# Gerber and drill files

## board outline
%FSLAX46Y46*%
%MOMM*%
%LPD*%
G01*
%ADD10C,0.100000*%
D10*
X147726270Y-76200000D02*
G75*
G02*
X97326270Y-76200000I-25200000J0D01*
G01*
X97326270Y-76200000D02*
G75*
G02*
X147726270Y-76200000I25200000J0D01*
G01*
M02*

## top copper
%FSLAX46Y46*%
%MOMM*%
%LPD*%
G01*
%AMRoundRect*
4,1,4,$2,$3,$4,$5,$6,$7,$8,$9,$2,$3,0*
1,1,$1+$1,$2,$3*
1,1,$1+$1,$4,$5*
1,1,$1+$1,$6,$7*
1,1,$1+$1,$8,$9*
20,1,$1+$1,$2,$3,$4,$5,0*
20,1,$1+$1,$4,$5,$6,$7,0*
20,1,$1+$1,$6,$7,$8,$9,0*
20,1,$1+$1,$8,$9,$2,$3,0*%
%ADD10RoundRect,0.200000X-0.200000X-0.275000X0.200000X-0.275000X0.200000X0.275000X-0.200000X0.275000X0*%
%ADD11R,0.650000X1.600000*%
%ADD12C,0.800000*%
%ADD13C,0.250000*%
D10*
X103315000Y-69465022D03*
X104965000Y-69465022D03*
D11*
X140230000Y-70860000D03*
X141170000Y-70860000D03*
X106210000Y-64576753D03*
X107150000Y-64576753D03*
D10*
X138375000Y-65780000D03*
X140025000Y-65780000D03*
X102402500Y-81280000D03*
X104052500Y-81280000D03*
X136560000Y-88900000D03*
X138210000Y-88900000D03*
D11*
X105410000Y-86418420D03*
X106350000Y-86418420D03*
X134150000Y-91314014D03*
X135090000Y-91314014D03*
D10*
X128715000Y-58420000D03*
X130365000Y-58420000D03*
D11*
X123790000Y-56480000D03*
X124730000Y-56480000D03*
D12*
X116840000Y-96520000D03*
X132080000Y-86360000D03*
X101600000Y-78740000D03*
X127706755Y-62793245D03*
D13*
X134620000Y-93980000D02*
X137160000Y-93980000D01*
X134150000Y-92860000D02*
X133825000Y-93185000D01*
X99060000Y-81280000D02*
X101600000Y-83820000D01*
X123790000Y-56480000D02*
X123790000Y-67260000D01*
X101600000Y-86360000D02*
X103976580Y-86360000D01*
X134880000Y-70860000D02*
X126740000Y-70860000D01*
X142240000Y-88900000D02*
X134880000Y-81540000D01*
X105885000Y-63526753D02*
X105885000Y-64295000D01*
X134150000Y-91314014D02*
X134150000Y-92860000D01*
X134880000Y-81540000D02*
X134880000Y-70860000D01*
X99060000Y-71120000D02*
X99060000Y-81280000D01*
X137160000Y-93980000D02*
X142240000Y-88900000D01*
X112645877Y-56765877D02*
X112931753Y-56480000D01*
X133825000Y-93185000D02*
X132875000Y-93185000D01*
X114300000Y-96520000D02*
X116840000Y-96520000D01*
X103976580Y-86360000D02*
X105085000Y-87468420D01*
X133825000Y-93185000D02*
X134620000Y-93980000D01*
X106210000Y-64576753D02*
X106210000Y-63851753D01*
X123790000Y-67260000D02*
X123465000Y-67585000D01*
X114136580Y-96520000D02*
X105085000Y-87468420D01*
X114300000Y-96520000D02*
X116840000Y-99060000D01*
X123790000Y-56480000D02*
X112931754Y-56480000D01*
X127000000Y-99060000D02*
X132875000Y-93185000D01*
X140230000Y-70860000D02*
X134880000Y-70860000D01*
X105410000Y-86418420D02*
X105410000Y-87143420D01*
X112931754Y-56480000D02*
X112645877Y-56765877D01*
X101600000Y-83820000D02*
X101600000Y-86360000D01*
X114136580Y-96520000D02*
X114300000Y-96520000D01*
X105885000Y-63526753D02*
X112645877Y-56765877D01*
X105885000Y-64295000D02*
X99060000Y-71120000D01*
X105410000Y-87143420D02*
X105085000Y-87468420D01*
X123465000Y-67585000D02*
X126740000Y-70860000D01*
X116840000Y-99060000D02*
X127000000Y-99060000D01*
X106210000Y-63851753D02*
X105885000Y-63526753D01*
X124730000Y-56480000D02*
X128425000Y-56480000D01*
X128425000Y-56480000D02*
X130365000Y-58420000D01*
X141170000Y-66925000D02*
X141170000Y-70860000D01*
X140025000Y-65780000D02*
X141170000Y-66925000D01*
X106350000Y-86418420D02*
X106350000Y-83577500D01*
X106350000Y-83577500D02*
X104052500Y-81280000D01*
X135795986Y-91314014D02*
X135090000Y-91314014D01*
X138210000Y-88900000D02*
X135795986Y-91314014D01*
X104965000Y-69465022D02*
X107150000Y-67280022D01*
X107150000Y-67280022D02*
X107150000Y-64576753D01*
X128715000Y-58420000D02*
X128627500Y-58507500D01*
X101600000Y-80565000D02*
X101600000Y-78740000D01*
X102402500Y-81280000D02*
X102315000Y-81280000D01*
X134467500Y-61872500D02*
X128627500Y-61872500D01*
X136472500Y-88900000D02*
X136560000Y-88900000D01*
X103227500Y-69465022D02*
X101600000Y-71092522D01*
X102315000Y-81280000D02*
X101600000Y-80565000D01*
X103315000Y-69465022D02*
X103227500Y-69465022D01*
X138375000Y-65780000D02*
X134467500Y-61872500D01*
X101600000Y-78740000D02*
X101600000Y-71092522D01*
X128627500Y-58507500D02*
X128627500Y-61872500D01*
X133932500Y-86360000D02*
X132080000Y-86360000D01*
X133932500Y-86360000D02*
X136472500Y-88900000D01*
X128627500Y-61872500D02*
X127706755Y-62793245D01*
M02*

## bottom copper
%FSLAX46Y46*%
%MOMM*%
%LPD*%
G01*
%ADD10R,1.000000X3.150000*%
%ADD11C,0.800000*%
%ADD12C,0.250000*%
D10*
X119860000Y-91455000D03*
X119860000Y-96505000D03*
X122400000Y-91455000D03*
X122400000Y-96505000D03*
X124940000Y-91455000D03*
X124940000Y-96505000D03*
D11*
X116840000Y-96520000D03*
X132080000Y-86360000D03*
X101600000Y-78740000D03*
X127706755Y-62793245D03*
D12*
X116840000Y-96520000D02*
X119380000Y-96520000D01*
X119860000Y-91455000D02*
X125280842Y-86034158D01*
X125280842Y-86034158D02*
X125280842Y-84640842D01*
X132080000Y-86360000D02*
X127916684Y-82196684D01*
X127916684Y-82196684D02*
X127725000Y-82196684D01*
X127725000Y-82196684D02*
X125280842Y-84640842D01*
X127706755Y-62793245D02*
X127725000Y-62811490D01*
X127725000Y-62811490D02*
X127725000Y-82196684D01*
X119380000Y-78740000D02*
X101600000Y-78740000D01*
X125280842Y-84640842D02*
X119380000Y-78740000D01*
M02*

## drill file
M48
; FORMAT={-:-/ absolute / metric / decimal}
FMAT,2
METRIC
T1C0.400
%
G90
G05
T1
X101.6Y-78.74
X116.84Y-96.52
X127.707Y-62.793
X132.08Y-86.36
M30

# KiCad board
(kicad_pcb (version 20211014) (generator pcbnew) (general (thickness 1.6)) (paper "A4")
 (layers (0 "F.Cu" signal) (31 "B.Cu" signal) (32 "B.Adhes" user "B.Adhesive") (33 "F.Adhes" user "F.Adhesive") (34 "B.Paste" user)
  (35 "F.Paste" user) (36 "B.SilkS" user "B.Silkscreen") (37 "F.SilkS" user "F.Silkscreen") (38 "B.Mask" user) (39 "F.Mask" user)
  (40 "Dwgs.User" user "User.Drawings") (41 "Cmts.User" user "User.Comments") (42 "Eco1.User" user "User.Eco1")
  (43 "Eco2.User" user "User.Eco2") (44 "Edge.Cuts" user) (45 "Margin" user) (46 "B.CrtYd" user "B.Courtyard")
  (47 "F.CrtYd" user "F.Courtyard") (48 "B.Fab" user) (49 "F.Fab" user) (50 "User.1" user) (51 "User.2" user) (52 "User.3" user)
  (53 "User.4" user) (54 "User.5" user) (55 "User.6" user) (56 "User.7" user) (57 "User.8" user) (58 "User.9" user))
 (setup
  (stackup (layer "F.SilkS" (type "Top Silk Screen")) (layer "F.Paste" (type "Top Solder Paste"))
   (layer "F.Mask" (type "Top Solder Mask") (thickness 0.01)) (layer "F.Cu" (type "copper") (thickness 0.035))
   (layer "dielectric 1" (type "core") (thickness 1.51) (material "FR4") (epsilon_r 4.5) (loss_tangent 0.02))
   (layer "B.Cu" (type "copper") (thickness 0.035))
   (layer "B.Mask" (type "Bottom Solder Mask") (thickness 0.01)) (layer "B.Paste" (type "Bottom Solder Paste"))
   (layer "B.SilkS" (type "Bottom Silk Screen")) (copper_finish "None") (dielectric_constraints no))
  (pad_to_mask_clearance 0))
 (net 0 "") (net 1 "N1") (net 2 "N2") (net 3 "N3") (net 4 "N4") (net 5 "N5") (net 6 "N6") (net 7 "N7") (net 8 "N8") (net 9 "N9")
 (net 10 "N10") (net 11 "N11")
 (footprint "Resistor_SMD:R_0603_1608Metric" (layer "F.Cu") (at 104.14 69.465022)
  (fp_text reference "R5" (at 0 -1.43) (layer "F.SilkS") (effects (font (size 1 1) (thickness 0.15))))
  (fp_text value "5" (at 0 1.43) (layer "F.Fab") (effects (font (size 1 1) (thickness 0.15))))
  (pad "1" smd roundrect (at -0.825 0) (size 0.8 0.95) (layers "F.Cu" "F.Paste" "F.Mask") (roundrect_rratio 0.25) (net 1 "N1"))
  (pad "2" smd roundrect (at 0.825 0) (size 0.8 0.95) (layers "F.Cu" "F.Paste" "F.Mask") (roundrect_rratio 0.25) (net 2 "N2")))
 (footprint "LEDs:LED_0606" (layer "F.Cu") (at 140.7 70.86)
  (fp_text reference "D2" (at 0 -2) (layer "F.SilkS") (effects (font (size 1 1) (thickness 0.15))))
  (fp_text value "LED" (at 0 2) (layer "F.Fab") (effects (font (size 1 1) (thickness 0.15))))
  (pad "1" smd rect locked (at -0.47 0 180) (size 0.65 1.6) (layers "F.Cu" "F.Paste" "F.Mask") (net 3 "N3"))
  (pad "2" smd rect locked (at 0.47 0 180) (size 0.65 1.6) (layers "F.Cu" "F.Paste" "F.Mask") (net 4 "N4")))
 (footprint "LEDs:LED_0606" (layer "F.Cu") (at 106.68 64.576753)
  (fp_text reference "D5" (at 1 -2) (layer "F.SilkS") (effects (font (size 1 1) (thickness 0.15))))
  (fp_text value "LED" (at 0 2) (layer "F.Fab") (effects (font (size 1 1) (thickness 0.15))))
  (pad "1" smd rect locked (at -0.47 0 180) (size 0.65 1.6) (layers "F.Cu" "F.Paste" "F.Mask") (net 3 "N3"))
  (pad "2" smd rect locked (at 0.47 0 180) (size 0.65 1.6) (layers "F.Cu" "F.Paste" "F.Mask") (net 2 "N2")))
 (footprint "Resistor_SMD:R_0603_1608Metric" (layer "F.Cu") (at 139.2 65.78)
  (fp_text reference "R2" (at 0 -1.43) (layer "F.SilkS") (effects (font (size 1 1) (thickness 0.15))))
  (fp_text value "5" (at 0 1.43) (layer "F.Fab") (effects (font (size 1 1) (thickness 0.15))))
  (pad "1" smd roundrect (at -0.825 0) (size 0.8 0.95) (layers "F.Cu" "F.Paste" "F.Mask") (roundrect_rratio 0.25) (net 1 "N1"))
  (pad "2" smd roundrect (at 0.825 0) (size 0.8 0.95) (layers "F.Cu" "F.Paste" "F.Mask") (roundrect_rratio 0.25) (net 4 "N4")))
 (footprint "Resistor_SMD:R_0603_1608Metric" (layer "F.Cu") (at 103.2275 81.28)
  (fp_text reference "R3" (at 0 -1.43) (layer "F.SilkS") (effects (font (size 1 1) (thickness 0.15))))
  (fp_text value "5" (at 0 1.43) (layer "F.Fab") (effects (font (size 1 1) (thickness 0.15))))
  (pad "1" smd roundrect (at -0.825 0) (size 0.8 0.95) (layers "F.Cu" "F.Paste" "F.Mask") (roundrect_rratio 0.25) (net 1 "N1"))
  (pad "2" smd roundrect (at 0.825 0) (size 0.8 0.95) (layers "F.Cu" "F.Paste" "F.Mask") (roundrect_rratio 0.25) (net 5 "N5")))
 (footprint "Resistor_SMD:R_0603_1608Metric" (layer "F.Cu") (at 137.385 88.9)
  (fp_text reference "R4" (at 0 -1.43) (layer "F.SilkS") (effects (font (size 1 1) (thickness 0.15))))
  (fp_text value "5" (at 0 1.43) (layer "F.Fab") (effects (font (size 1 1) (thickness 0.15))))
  (pad "1" smd roundrect (at -0.825 0) (size 0.8 0.95) (layers "F.Cu" "F.Paste" "F.Mask") (roundrect_rratio 0.25) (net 1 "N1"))
  (pad "2" smd roundrect (at 0.825 0) (size 0.8 0.95) (layers "F.Cu" "F.Paste" "F.Mask") (roundrect_rratio 0.25) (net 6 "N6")))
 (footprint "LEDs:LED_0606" (layer "F.Cu") (at 105.88 86.41842)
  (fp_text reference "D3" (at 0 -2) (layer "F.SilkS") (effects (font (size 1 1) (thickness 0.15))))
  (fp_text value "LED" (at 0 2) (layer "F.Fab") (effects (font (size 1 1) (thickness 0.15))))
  (pad "1" smd rect locked (at -0.47 0 180) (size 0.65 1.6) (layers "F.Cu" "F.Paste" "F.Mask") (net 3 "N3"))
  (pad "2" smd rect locked (at 0.47 0 180) (size 0.65 1.6) (layers "F.Cu" "F.Paste" "F.Mask") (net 5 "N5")))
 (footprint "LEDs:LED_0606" (layer "F.Cu") (at 134.62 91.314014)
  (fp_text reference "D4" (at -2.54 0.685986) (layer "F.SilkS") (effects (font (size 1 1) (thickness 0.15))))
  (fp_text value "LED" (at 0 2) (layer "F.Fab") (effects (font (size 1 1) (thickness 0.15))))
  (pad "1" smd rect locked (at -0.47 0 180) (size 0.65 1.6) (layers "F.Cu" "F.Paste" "F.Mask") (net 3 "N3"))
  (pad "2" smd rect locked (at 0.47 0 180) (size 0.65 1.6) (layers "F.Cu" "F.Paste" "F.Mask") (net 6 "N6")))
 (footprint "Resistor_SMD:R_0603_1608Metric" (layer "F.Cu") (at 129.54 58.42)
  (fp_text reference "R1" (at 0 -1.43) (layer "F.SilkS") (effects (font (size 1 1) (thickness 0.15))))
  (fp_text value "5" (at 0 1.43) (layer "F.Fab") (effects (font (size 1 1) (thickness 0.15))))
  (pad "1" smd roundrect (at -0.825 0) (size 0.8 0.95) (layers "F.Cu" "F.Paste" "F.Mask") (roundrect_rratio 0.25) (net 1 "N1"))
  (pad "2" smd roundrect (at 0.825 0) (size 0.8 0.95) (layers "F.Cu" "F.Paste" "F.Mask") (roundrect_rratio 0.25) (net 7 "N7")))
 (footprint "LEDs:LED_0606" (layer "F.Cu") (at 124.26 56.48)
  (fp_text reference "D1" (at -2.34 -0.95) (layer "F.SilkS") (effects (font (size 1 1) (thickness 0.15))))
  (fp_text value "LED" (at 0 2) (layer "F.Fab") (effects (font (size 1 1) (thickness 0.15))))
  (pad "1" smd rect locked (at -0.47 0 180) (size 0.65 1.6) (layers "F.Cu" "F.Paste" "F.Mask") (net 3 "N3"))
  (pad "2" smd rect locked (at 0.47 0 180) (size 0.65 1.6) (layers "F.Cu" "F.Paste" "F.Mask") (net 7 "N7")))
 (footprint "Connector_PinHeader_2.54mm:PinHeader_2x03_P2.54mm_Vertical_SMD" (layer "B.Cu") (at 122.4 93.98 -90)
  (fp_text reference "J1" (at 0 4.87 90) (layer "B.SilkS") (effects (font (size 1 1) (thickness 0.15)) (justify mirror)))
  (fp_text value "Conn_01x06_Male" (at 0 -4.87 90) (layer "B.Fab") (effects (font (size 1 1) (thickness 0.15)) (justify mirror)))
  (pad "1" smd rect (at -2.525 2.54 270) (size 3.15 1) (layers "B.Cu" "B.Paste" "B.Mask") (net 1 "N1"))
  (pad "2" smd rect (at 2.525 2.54 270) (size 3.15 1) (layers "B.Cu" "B.Paste" "B.Mask") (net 3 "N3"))
  (pad "3" smd rect (at -2.525 0 270) (size 3.15 1) (layers "B.Cu" "B.Paste" "B.Mask") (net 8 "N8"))
  (pad "4" smd rect (at 2.525 0 270) (size 3.15 1) (layers "B.Cu" "B.Paste" "B.Mask") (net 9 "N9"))
  (pad "5" smd rect (at -2.525 -2.54 270) (size 3.15 1) (layers "B.Cu" "B.Paste" "B.Mask") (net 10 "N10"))
  (pad "6" smd rect (at 2.525 -2.54 270) (size 3.15 1) (layers "B.Cu" "B.Paste" "B.Mask") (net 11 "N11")))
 (gr_circle (center 122.52627 76.2) (end 147.72627 76.2) (layer "Edge.Cuts") (width 0.1) (fill none))
 (segment (start 134.62 93.98) (end 137.16 93.98) (width 0.25) (layer "F.Cu") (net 3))
 (segment (start 134.15 92.86) (end 133.825 93.185) (width 0.25) (layer "F.Cu") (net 3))
 (segment (start 99.06 81.28) (end 101.6 83.82) (width 0.25) (layer "F.Cu") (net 3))
 (segment (start 123.79 56.48) (end 123.79 67.26) (width 0.25) (layer "F.Cu") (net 3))
 (segment (start 101.6 86.36) (end 103.97658 86.36) (width 0.25) (layer "F.Cu") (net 3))
 (segment (start 134.88 70.86) (end 126.74 70.86) (width 0.25) (layer "F.Cu") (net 3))
 (segment (start 142.24 88.9) (end 134.88 81.54) (width 0.25) (layer "F.Cu") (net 3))
 (segment (start 105.885 63.526753) (end 105.885 64.295) (width 0.25) (layer "F.Cu") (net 3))
 (segment (start 134.15 91.314014) (end 134.15 92.86) (width 0.25) (layer "F.Cu") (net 3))
 (segment (start 134.88 81.54) (end 134.88 70.86) (width 0.25) (layer "F.Cu") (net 3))
 (segment (start 99.06 71.12) (end 99.06 81.28) (width 0.25) (layer "F.Cu") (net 3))
 (segment (start 137.16 93.98) (end 142.24 88.9) (width 0.25) (layer "F.Cu") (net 3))
 (segment (start 112.645877 56.765877) (end 112.931753 56.48) (width 0.25) (layer "F.Cu") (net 3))
 (segment (start 133.825 93.185) (end 132.875 93.185) (width 0.25) (layer "F.Cu") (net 3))
 (segment (start 114.3 96.52) (end 116.84 96.52) (width 0.25) (layer "F.Cu") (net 3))
 (segment (start 103.97658 86.36) (end 105.085 87.46842) (width 0.25) (layer "F.Cu") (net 3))
 (segment (start 133.825 93.185) (end 134.62 93.98) (width 0.25) (layer "F.Cu") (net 3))
 (segment (start 106.21 64.576753) (end 106.21 63.851753) (width 0.25) (layer "F.Cu") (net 3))
 (segment (start 123.79 67.26) (end 123.465 67.585) (width 0.25) (layer "F.Cu") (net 3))
 (segment (start 114.13658 96.52) (end 105.085 87.46842) (width 0.25) (layer "F.Cu") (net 3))
 (segment (start 114.3 96.52) (end 116.84 99.06) (width 0.25) (layer "F.Cu") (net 3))
 (segment (start 123.79 56.48) (end 112.931754 56.48) (width 0.25) (layer "F.Cu") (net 3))
 (segment (start 127 99.06) (end 132.875 93.185) (width 0.25) (layer "F.Cu") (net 3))
 (segment (start 140.23 70.86) (end 134.88 70.86) (width 0.25) (layer "F.Cu") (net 3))
 (segment (start 105.41 86.41842) (end 105.41 87.14342) (width 0.25) (layer "F.Cu") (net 3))
 (segment (start 112.931754 56.48) (end 112.645877 56.765877) (width 0.25) (layer "F.Cu") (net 3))
 (segment (start 101.6 83.82) (end 101.6 86.36) (width 0.25) (layer "F.Cu") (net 3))
 (segment (start 114.13658 96.52) (end 114.3 96.52) (width 0.25) (layer "F.Cu") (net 3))
 (segment (start 105.885 63.526753) (end 112.645877 56.765877) (width 0.25) (layer "F.Cu") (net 3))
 (segment (start 105.885 64.295) (end 99.06 71.12) (width 0.25) (layer "F.Cu") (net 3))
 (segment (start 105.41 87.14342) (end 105.085 87.46842) (width 0.25) (layer "F.Cu") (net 3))
 (segment (start 123.465 67.585) (end 126.74 70.86) (width 0.25) (layer "F.Cu") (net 3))
 (segment (start 116.84 99.06) (end 127 99.06) (width 0.25) (layer "F.Cu") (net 3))
 (segment (start 106.21 63.851753) (end 105.885 63.526753) (width 0.25) (layer "F.Cu") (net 3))
 (via (at 116.84 96.52) (size 0.8) (drill 0.4) (layers "F.Cu" "B.Cu") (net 3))
 (segment (start 116.84 96.52) (end 119.38 96.52) (width 0.25) (layer "B.Cu") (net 3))
 (segment (start 124.73 56.48) (end 128.425 56.48) (width 0.25) (layer "F.Cu") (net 7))
 (segment (start 128.425 56.48) (end 130.365 58.42) (width 0.25) (layer "F.Cu") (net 7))
 (segment (start 141.17 66.925) (end 141.17 70.86) (width 0.25) (layer "F.Cu") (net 4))
 (segment (start 140.025 65.78) (end 141.17 66.925) (width 0.25) (layer "F.Cu") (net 4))
 (segment (start 106.35 86.41842) (end 106.35 83.5775) (width 0.25) (layer "F.Cu") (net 5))
 (segment (start 106.35 83.5775) (end 104.0525 81.28) (width 0.25) (layer "F.Cu") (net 5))
 (segment (start 135.795986 91.314014) (end 135.09 91.314014) (width 0.25) (layer "F.Cu") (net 6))
 (segment (start 138.21 88.9) (end 135.795986 91.314014) (width 0.25) (layer "F.Cu") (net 6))
 (segment (start 104.965 69.465022) (end 107.15 67.280022) (width 0.25) (layer "F.Cu") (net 2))
 (segment (start 107.15 67.280022) (end 107.15 64.576753) (width 0.25) (layer "F.Cu") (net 2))
 (segment (start 128.715 58.42) (end 128.6275 58.5075) (width 0.25) (layer "F.Cu") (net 1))
 (segment (start 101.6 80.565) (end 101.6 78.74) (width 0.25) (layer "F.Cu") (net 1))
 (segment (start 102.4025 81.28) (end 102.315 81.28) (width 0.25) (layer "F.Cu") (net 1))
 (segment (start 134.4675 61.8725) (end 128.6275 61.8725) (width 0.25) (layer "F.Cu") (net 1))
 (segment (start 136.4725 88.9) (end 136.56 88.9) (width 0.25) (layer "F.Cu") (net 1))
 (segment (start 103.2275 69.465022) (end 101.6 71.092522) (width 0.25) (layer "F.Cu") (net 1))
 (segment (start 102.315 81.28) (end 101.6 80.565) (width 0.25) (layer "F.Cu") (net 1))
 (segment (start 103.315 69.465022) (end 103.2275 69.465022) (width 0.25) (layer "F.Cu") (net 1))
 (segment (start 138.375 65.78) (end 134.4675 61.8725) (width 0.25) (layer "F.Cu") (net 1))
 (segment (start 101.6 78.74) (end 101.6 71.092522) (width 0.25) (layer "F.Cu") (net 1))
 (segment (start 128.6275 58.5075) (end 128.6275 61.8725) (width 0.25) (layer "F.Cu") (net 1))
 (segment (start 133.9325 86.36) (end 132.08 86.36) (width 0.25) (layer "F.Cu") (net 1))
 (segment (start 133.9325 86.36) (end 136.4725 88.9) (width 0.25) (layer "F.Cu") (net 1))
 (segment (start 128.6275 61.8725) (end 127.706755 62.793245) (width 0.25) (layer "F.Cu") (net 1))
 (via (at 132.08 86.36) (size 0.8) (drill 0.4) (layers "F.Cu" "B.Cu") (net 1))
 (via (at 101.6 78.74) (size 0.8) (drill 0.4) (layers "F.Cu" "B.Cu") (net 1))
 (via (at 127.706755 62.793245) (size 0.8) (drill 0.4) (layers "F.Cu" "B.Cu") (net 1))
 (segment (start 119.86 91.455) (end 125.280842 86.034158) (width 0.25) (layer "B.Cu") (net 1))
 (segment (start 125.280842 86.034158) (end 125.280842 84.640842) (width 0.25) (layer "B.Cu") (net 1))
 (segment (start 132.08 86.36) (end 127.916684 82.196684) (width 0.25) (layer "B.Cu") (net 1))
 (segment (start 127.916684 82.196684) (end 127.725 82.196684) (width 0.25) (layer "B.Cu") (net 1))
 (segment (start 127.725 82.196684) (end 125.280842 84.640842) (width 0.25) (layer "B.Cu") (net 1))
 (segment (start 127.706755 62.793245) (end 127.725 62.81149) (width 0.25) (layer "B.Cu") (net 1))
 (segment (start 127.725 62.81149) (end 127.725 82.196684) (width 0.25) (layer "B.Cu") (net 1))
 (segment (start 119.38 78.74) (end 101.6 78.74) (width 0.25) (layer "B.Cu") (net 1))
 (segment (start 125.280842 84.640842) (end 119.38 78.74) (width 0.25) (layer "B.Cu") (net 1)))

